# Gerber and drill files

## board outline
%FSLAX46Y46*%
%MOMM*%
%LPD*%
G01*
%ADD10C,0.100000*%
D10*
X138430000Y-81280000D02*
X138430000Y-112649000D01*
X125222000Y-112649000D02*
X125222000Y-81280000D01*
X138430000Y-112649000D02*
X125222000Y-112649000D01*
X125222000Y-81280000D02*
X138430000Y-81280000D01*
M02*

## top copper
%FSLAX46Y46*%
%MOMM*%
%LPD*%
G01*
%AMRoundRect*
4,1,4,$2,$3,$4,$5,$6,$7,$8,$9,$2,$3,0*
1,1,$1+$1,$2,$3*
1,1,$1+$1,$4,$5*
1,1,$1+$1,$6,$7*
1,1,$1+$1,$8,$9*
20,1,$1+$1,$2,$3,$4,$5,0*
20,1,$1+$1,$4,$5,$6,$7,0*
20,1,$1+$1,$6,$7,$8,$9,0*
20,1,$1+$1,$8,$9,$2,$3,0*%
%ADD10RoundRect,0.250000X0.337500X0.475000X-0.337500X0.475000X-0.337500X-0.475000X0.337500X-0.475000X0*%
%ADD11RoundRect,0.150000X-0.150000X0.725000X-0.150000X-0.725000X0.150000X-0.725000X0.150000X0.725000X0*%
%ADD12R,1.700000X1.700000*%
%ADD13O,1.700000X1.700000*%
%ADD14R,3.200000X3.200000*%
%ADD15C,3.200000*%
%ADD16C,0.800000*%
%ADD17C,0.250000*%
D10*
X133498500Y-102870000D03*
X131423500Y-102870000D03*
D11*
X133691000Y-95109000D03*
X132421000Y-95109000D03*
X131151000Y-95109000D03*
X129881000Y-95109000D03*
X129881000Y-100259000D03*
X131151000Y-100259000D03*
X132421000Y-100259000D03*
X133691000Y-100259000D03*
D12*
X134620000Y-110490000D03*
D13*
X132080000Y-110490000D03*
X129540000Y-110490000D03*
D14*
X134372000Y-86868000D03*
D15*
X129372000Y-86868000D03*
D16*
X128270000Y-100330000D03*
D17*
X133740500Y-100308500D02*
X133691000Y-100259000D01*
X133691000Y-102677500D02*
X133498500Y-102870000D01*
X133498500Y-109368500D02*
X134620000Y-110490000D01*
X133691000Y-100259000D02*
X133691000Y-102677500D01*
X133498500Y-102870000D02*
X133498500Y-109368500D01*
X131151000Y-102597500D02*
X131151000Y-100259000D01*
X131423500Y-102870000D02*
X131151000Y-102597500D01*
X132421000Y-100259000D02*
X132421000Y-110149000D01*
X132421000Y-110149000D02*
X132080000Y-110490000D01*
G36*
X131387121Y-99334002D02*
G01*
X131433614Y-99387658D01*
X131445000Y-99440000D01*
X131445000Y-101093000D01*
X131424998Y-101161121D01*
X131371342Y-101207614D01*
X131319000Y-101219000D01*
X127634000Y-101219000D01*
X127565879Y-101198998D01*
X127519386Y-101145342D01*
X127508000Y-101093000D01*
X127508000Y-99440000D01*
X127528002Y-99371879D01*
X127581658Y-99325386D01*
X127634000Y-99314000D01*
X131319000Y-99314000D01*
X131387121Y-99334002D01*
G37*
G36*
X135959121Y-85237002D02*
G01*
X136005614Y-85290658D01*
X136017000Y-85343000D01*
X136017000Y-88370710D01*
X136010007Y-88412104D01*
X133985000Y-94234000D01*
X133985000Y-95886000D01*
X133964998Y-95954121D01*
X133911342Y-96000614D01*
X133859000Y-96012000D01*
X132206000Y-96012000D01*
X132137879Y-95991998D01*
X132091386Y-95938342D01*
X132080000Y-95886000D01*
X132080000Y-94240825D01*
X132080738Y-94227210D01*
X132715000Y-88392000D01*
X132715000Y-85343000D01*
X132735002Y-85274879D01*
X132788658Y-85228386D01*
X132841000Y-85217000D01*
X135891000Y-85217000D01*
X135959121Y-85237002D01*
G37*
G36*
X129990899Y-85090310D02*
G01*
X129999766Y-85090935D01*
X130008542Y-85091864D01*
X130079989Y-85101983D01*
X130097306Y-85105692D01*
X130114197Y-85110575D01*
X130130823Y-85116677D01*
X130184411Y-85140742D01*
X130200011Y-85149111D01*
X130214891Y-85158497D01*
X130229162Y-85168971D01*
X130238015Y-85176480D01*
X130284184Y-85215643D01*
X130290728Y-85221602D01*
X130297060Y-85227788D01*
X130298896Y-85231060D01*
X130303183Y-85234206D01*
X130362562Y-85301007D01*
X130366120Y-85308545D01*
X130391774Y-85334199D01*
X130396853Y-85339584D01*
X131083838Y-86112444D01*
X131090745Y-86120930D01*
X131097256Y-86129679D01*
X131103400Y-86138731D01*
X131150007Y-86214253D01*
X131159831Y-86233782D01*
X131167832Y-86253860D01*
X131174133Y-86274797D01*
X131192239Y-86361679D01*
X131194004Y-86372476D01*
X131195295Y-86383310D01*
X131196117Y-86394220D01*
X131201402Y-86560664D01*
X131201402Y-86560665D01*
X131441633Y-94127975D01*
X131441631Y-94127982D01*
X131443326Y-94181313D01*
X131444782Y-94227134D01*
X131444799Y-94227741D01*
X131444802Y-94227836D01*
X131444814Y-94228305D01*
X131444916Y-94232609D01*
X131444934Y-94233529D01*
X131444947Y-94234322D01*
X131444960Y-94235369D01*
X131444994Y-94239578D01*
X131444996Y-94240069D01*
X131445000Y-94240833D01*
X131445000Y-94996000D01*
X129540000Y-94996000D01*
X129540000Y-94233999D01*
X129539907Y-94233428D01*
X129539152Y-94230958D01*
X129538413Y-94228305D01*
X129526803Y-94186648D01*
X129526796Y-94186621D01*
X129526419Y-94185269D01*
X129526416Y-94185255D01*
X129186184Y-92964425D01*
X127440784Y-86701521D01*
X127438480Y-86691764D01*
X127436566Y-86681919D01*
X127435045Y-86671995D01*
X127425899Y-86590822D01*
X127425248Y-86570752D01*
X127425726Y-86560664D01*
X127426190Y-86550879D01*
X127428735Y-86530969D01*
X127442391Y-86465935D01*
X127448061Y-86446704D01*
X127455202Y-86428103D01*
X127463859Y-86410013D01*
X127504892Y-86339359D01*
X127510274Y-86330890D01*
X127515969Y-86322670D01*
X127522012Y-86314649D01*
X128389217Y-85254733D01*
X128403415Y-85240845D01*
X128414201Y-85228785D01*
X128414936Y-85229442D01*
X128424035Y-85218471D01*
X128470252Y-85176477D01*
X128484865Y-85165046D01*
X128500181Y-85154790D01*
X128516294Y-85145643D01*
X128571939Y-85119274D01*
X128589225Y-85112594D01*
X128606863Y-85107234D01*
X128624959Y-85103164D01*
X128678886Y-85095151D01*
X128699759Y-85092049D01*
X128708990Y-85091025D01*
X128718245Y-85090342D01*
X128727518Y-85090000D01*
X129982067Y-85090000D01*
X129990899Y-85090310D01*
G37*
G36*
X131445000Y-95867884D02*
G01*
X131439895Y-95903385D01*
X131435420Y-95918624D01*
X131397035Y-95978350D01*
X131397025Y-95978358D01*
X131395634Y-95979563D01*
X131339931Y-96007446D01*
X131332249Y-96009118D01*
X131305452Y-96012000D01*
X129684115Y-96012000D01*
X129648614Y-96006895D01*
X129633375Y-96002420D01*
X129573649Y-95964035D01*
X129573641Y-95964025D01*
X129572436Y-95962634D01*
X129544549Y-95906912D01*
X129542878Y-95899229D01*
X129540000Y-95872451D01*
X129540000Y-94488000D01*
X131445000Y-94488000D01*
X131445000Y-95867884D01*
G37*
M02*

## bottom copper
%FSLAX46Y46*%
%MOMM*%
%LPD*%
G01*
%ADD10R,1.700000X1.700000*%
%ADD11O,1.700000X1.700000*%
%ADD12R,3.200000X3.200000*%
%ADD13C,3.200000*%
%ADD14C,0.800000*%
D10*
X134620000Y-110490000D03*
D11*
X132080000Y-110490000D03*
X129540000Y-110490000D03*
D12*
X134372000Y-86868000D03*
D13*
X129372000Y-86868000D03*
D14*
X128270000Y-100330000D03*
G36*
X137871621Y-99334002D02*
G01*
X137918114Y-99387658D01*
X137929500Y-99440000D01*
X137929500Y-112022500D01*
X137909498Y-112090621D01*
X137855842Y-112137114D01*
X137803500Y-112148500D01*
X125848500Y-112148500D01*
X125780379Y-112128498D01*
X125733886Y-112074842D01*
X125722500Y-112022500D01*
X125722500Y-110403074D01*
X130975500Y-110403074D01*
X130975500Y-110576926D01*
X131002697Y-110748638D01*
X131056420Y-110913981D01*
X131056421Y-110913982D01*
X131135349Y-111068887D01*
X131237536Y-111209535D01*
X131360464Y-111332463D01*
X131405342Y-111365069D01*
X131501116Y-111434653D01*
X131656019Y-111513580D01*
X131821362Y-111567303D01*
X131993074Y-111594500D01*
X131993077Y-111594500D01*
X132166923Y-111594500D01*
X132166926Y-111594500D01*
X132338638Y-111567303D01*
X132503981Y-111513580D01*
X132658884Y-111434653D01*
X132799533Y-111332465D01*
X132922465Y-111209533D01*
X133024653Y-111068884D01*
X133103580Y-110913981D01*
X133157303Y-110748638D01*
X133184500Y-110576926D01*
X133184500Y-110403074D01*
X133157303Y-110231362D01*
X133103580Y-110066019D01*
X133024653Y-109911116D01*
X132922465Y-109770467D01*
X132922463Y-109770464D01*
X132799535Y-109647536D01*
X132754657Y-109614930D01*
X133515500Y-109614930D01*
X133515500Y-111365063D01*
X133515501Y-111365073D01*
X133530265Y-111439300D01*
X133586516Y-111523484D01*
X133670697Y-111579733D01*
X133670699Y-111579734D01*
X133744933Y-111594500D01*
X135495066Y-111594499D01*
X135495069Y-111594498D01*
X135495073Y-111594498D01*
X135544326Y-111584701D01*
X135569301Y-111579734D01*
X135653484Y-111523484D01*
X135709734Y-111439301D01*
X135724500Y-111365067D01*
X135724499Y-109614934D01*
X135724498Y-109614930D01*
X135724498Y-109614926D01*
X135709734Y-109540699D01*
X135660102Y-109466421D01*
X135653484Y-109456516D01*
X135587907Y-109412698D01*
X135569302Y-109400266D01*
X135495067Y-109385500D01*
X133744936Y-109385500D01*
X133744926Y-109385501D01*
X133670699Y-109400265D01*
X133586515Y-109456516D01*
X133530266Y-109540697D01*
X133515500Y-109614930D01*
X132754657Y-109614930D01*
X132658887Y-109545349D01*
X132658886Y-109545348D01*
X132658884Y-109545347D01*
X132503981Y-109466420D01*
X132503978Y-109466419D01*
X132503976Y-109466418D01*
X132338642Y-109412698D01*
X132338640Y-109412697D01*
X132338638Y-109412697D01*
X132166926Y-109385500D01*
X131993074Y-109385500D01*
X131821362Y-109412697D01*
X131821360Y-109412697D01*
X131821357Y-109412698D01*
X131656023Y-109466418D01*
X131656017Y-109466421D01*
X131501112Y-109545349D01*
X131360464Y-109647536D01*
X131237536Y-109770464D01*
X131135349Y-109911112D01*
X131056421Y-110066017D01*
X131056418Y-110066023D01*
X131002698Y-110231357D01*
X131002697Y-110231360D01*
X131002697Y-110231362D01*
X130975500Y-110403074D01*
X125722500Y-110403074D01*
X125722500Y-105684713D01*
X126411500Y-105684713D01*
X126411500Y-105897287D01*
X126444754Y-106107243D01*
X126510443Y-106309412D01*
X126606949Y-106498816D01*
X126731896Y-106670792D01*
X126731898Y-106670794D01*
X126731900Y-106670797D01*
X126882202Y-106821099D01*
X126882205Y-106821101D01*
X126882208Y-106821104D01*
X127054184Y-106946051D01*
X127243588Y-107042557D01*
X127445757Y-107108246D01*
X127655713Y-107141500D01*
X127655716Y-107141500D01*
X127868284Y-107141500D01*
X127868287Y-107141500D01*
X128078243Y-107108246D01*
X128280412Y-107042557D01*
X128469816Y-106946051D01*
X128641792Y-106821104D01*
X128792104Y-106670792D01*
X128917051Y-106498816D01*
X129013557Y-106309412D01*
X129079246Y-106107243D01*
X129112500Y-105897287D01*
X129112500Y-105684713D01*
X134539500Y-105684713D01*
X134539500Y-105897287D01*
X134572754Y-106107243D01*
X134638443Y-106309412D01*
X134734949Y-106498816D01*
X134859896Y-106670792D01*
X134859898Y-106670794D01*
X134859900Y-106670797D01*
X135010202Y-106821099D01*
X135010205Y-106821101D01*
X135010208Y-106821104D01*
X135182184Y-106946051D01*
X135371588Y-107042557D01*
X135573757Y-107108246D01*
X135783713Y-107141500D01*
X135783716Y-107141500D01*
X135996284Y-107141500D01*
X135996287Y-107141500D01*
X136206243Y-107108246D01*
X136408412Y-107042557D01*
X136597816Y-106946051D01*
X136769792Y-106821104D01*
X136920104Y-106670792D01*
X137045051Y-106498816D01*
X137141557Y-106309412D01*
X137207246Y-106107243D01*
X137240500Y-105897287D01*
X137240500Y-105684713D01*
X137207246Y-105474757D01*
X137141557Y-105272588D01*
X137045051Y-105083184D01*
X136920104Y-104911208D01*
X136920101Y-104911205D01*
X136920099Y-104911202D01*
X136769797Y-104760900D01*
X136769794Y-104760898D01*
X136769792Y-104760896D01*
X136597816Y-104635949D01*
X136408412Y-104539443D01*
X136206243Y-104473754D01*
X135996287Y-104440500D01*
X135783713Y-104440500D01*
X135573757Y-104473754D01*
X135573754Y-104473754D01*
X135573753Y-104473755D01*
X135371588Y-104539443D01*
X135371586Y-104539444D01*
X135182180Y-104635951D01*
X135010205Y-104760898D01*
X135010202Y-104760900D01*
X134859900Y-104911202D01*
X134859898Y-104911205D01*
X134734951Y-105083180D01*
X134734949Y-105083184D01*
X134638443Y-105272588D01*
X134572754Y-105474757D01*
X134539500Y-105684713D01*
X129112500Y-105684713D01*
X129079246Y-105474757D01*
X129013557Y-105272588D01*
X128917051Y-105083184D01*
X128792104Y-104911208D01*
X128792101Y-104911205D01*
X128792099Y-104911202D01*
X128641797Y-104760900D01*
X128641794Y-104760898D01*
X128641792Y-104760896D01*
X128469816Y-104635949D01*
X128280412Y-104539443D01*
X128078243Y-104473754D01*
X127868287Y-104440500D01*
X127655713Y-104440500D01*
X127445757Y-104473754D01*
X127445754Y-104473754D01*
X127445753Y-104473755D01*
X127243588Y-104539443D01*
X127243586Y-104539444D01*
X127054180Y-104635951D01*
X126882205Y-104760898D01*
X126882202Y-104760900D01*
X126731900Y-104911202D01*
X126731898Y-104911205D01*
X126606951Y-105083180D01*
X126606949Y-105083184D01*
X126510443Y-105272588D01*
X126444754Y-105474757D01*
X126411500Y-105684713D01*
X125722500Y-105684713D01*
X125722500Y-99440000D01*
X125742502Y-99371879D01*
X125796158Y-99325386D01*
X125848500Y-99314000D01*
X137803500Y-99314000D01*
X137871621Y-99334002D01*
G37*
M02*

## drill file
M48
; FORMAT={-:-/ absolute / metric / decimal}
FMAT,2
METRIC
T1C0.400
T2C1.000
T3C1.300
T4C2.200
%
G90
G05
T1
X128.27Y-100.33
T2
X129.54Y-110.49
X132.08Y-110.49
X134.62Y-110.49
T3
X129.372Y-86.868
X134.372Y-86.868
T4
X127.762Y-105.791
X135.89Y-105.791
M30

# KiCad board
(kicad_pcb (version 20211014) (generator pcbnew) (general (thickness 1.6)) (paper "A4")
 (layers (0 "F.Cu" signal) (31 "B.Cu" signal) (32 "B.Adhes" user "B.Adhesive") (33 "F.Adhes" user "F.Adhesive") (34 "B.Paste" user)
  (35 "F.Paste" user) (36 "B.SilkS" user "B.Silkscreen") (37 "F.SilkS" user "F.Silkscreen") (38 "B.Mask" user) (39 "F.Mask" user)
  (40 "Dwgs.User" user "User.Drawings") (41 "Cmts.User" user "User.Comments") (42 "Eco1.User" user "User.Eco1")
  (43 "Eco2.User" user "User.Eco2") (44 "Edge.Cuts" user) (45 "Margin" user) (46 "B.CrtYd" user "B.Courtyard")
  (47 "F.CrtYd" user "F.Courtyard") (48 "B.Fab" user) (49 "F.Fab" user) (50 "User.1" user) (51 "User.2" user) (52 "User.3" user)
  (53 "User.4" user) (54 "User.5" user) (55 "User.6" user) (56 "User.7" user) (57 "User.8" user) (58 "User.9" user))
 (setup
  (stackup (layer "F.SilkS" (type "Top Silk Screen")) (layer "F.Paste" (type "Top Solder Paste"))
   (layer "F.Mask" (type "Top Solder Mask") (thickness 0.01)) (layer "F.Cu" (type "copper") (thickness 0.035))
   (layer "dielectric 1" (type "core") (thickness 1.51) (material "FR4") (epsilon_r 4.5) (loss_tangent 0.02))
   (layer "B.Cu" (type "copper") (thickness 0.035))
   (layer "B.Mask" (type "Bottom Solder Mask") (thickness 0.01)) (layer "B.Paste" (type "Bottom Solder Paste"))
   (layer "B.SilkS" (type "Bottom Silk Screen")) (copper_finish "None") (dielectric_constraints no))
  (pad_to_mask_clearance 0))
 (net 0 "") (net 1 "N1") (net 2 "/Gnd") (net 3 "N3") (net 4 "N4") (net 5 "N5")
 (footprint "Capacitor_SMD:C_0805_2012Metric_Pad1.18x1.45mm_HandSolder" (layer "F.Cu") (at 132.461 102.87 180)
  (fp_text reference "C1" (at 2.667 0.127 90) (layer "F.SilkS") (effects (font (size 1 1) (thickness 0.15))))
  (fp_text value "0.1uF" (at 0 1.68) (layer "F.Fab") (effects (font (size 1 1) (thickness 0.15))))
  (pad "1" smd roundrect (at -1.0375 0 180) (size 1.175 1.45) (layers "F.Cu" "F.Paste" "F.Mask") (roundrect_rratio 0.2127659574)
   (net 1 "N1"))
  (pad "2" smd roundrect (at 1.0375 0 180) (size 1.175 1.45) (layers "F.Cu" "F.Paste" "F.Mask") (roundrect_rratio 0.2127659574)
   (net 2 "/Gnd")))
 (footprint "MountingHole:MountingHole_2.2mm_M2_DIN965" (layer "F.Cu") (at 135.89 105.791)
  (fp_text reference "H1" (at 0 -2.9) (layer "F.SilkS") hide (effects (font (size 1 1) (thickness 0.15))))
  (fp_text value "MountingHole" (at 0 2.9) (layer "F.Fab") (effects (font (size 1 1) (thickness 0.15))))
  (pad "" np_thru_hole circle (at 0 0) (size 2.2 2.2) (drill 2.2) (layers *.Cu *.Mask)))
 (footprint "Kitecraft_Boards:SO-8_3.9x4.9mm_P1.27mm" (layer "F.Cu") (at 131.786 97.684 -90)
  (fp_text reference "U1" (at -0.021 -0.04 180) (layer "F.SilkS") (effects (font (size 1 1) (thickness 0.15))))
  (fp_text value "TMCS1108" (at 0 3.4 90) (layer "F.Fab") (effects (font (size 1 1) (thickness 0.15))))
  (pad "1" smd roundrect (at -2.575 -1.905 270) (size 1.75 0.6) (layers "F.Cu" "F.Paste" "F.Mask") (roundrect_rratio 0.25) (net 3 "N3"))
  (pad "2" smd roundrect (at -2.575 -0.635 270) (size 1.75 0.6) (layers "F.Cu" "F.Paste" "F.Mask") (roundrect_rratio 0.25) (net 3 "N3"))
  (pad "3" smd roundrect (at -2.575 0.635 270) (size 1.75 0.6) (layers "F.Cu" "F.Paste" "F.Mask") (roundrect_rratio 0.25) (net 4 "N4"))
  (pad "4" smd roundrect (at -2.575 1.905 270) (size 1.75 0.6) (layers "F.Cu" "F.Paste" "F.Mask") (roundrect_rratio 0.25) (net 4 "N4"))
  (pad "5" smd roundrect (at 2.575 1.905 270) (size 1.75 0.6) (layers "F.Cu" "F.Paste" "F.Mask") (roundrect_rratio 0.25) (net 2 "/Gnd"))
  (pad "6" smd roundrect (at 2.575 0.635 270) (size 1.75 0.6) (layers "F.Cu" "F.Paste" "F.Mask") (roundrect_rratio 0.25) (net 2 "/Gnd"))
  (pad "7" smd roundrect (at 2.575 -0.635 270) (size 1.75 0.6) (layers "F.Cu" "F.Paste" "F.Mask") (roundrect_rratio 0.25) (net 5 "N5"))
  (pad "8" smd roundrect (at 2.575 -1.905 270) (size 1.75 0.6) (layers "F.Cu" "F.Paste" "F.Mask") (roundrect_rratio 0.25) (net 1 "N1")))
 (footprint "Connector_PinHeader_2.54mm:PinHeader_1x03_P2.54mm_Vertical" (layer "F.Cu") (at 134.62 110.49 -90)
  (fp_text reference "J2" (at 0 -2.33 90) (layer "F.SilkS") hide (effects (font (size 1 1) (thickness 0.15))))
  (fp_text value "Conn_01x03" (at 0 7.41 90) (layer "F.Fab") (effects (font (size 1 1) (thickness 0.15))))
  (pad "1" thru_hole rect (at 0 0 270) (size 1.7 1.7) (drill 1) (layers *.Cu *.Mask) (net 1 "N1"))
  (pad "2" thru_hole oval (at 0 2.54 270) (size 1.7 1.7) (drill 1) (layers *.Cu *.Mask) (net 5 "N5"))
  (pad "3" thru_hole oval (at 0 5.08 270) (size 1.7 1.7) (drill 1) (layers *.Cu *.Mask) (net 2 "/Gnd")))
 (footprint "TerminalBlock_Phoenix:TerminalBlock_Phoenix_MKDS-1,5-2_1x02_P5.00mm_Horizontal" (layer "F.Cu") (at 134.372 86.868 180)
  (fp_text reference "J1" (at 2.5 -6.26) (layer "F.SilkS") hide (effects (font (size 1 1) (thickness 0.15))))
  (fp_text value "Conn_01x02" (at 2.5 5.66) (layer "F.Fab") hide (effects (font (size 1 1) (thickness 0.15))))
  (pad "1" thru_hole rect (at 0 0 180) (size 3.2 3.2) (drill 1.3) (layers *.Cu *.Mask) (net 3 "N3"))
  (pad "2" thru_hole circle (at 5 0 180) (size 3.2 3.2) (drill 1.3) (layers *.Cu *.Mask) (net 4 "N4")))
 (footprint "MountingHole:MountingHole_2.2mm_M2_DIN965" (layer "F.Cu") (at 127.762 105.791)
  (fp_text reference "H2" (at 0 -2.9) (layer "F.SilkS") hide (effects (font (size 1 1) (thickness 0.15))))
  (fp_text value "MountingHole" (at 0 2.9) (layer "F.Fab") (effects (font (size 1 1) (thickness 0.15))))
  (pad "" np_thru_hole circle (at 0 0) (size 2.2 2.2) (drill 2.2) (layers *.Cu *.Mask)))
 (gr_line (start 138.43 81.28) (end 138.43 112.649) (layer "Edge.Cuts") (width 0.1))
 (gr_line (start 125.222 112.649) (end 125.222 81.28) (layer "Edge.Cuts") (width 0.1))
 (gr_line (start 138.43 112.649) (end 125.222 112.649) (layer "Edge.Cuts") (width 0.1))
 (gr_line (start 125.222 81.28) (end 138.43 81.28) (layer "Edge.Cuts") (width 0.1))
 (segment (start 133.7405 100.3085) (end 133.691 100.259) (width 0.25) (layer "F.Cu") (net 1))
 (segment (start 133.691 102.6775) (end 133.4985 102.87) (width 0.25) (layer "F.Cu") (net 1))
 (segment (start 133.4985 109.3685) (end 134.62 110.49) (width 0.25) (layer "F.Cu") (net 1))
 (segment (start 133.691 100.259) (end 133.691 102.6775) (width 0.25) (layer "F.Cu") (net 1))
 (segment (start 133.4985 102.87) (end 133.4985 109.3685) (width 0.25) (layer "F.Cu") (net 1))
 (segment (start 131.151 102.5975) (end 131.151 100.259) (width 0.25) (layer "F.Cu") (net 2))
 (segment (start 131.4235 102.87) (end 131.151 102.5975) (width 0.25) (layer "F.Cu") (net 2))
 (via (at 128.27 100.33) (size 0.8) (drill 0.4) (layers "F.Cu" "B.Cu") (free) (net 2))
 (segment (start 132.421 100.259) (end 132.421 110.149) (width 0.25) (layer "F.Cu") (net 5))
 (segment (start 132.421 110.149) (end 132.08 110.49) (width 0.25) (layer "F.Cu") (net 5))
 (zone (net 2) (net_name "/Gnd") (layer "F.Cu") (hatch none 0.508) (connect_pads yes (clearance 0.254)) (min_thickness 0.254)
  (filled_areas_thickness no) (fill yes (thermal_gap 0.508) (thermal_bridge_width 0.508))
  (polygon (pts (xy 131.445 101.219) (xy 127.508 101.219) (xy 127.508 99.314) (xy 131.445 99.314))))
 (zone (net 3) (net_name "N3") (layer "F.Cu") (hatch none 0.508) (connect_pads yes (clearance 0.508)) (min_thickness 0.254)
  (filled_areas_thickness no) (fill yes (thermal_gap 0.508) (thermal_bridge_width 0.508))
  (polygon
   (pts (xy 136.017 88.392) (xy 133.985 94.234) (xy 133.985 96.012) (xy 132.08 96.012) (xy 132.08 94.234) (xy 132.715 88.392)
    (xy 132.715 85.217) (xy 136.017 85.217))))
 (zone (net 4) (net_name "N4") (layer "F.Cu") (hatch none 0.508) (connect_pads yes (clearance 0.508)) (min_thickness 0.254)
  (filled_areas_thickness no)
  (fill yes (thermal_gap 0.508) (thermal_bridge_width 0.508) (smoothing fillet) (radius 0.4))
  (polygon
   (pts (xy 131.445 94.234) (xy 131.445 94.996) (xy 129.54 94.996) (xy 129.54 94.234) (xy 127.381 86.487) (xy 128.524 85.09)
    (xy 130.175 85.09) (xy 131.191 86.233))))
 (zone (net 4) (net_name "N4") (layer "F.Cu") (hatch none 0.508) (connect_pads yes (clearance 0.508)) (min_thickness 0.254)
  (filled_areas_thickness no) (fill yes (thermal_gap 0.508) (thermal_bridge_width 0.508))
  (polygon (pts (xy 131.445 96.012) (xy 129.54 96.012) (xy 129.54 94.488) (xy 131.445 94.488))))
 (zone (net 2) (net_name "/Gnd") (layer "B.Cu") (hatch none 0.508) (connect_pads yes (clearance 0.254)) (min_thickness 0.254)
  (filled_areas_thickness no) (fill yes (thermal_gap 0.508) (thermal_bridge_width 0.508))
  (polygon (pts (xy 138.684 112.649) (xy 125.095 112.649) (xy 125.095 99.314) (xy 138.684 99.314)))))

